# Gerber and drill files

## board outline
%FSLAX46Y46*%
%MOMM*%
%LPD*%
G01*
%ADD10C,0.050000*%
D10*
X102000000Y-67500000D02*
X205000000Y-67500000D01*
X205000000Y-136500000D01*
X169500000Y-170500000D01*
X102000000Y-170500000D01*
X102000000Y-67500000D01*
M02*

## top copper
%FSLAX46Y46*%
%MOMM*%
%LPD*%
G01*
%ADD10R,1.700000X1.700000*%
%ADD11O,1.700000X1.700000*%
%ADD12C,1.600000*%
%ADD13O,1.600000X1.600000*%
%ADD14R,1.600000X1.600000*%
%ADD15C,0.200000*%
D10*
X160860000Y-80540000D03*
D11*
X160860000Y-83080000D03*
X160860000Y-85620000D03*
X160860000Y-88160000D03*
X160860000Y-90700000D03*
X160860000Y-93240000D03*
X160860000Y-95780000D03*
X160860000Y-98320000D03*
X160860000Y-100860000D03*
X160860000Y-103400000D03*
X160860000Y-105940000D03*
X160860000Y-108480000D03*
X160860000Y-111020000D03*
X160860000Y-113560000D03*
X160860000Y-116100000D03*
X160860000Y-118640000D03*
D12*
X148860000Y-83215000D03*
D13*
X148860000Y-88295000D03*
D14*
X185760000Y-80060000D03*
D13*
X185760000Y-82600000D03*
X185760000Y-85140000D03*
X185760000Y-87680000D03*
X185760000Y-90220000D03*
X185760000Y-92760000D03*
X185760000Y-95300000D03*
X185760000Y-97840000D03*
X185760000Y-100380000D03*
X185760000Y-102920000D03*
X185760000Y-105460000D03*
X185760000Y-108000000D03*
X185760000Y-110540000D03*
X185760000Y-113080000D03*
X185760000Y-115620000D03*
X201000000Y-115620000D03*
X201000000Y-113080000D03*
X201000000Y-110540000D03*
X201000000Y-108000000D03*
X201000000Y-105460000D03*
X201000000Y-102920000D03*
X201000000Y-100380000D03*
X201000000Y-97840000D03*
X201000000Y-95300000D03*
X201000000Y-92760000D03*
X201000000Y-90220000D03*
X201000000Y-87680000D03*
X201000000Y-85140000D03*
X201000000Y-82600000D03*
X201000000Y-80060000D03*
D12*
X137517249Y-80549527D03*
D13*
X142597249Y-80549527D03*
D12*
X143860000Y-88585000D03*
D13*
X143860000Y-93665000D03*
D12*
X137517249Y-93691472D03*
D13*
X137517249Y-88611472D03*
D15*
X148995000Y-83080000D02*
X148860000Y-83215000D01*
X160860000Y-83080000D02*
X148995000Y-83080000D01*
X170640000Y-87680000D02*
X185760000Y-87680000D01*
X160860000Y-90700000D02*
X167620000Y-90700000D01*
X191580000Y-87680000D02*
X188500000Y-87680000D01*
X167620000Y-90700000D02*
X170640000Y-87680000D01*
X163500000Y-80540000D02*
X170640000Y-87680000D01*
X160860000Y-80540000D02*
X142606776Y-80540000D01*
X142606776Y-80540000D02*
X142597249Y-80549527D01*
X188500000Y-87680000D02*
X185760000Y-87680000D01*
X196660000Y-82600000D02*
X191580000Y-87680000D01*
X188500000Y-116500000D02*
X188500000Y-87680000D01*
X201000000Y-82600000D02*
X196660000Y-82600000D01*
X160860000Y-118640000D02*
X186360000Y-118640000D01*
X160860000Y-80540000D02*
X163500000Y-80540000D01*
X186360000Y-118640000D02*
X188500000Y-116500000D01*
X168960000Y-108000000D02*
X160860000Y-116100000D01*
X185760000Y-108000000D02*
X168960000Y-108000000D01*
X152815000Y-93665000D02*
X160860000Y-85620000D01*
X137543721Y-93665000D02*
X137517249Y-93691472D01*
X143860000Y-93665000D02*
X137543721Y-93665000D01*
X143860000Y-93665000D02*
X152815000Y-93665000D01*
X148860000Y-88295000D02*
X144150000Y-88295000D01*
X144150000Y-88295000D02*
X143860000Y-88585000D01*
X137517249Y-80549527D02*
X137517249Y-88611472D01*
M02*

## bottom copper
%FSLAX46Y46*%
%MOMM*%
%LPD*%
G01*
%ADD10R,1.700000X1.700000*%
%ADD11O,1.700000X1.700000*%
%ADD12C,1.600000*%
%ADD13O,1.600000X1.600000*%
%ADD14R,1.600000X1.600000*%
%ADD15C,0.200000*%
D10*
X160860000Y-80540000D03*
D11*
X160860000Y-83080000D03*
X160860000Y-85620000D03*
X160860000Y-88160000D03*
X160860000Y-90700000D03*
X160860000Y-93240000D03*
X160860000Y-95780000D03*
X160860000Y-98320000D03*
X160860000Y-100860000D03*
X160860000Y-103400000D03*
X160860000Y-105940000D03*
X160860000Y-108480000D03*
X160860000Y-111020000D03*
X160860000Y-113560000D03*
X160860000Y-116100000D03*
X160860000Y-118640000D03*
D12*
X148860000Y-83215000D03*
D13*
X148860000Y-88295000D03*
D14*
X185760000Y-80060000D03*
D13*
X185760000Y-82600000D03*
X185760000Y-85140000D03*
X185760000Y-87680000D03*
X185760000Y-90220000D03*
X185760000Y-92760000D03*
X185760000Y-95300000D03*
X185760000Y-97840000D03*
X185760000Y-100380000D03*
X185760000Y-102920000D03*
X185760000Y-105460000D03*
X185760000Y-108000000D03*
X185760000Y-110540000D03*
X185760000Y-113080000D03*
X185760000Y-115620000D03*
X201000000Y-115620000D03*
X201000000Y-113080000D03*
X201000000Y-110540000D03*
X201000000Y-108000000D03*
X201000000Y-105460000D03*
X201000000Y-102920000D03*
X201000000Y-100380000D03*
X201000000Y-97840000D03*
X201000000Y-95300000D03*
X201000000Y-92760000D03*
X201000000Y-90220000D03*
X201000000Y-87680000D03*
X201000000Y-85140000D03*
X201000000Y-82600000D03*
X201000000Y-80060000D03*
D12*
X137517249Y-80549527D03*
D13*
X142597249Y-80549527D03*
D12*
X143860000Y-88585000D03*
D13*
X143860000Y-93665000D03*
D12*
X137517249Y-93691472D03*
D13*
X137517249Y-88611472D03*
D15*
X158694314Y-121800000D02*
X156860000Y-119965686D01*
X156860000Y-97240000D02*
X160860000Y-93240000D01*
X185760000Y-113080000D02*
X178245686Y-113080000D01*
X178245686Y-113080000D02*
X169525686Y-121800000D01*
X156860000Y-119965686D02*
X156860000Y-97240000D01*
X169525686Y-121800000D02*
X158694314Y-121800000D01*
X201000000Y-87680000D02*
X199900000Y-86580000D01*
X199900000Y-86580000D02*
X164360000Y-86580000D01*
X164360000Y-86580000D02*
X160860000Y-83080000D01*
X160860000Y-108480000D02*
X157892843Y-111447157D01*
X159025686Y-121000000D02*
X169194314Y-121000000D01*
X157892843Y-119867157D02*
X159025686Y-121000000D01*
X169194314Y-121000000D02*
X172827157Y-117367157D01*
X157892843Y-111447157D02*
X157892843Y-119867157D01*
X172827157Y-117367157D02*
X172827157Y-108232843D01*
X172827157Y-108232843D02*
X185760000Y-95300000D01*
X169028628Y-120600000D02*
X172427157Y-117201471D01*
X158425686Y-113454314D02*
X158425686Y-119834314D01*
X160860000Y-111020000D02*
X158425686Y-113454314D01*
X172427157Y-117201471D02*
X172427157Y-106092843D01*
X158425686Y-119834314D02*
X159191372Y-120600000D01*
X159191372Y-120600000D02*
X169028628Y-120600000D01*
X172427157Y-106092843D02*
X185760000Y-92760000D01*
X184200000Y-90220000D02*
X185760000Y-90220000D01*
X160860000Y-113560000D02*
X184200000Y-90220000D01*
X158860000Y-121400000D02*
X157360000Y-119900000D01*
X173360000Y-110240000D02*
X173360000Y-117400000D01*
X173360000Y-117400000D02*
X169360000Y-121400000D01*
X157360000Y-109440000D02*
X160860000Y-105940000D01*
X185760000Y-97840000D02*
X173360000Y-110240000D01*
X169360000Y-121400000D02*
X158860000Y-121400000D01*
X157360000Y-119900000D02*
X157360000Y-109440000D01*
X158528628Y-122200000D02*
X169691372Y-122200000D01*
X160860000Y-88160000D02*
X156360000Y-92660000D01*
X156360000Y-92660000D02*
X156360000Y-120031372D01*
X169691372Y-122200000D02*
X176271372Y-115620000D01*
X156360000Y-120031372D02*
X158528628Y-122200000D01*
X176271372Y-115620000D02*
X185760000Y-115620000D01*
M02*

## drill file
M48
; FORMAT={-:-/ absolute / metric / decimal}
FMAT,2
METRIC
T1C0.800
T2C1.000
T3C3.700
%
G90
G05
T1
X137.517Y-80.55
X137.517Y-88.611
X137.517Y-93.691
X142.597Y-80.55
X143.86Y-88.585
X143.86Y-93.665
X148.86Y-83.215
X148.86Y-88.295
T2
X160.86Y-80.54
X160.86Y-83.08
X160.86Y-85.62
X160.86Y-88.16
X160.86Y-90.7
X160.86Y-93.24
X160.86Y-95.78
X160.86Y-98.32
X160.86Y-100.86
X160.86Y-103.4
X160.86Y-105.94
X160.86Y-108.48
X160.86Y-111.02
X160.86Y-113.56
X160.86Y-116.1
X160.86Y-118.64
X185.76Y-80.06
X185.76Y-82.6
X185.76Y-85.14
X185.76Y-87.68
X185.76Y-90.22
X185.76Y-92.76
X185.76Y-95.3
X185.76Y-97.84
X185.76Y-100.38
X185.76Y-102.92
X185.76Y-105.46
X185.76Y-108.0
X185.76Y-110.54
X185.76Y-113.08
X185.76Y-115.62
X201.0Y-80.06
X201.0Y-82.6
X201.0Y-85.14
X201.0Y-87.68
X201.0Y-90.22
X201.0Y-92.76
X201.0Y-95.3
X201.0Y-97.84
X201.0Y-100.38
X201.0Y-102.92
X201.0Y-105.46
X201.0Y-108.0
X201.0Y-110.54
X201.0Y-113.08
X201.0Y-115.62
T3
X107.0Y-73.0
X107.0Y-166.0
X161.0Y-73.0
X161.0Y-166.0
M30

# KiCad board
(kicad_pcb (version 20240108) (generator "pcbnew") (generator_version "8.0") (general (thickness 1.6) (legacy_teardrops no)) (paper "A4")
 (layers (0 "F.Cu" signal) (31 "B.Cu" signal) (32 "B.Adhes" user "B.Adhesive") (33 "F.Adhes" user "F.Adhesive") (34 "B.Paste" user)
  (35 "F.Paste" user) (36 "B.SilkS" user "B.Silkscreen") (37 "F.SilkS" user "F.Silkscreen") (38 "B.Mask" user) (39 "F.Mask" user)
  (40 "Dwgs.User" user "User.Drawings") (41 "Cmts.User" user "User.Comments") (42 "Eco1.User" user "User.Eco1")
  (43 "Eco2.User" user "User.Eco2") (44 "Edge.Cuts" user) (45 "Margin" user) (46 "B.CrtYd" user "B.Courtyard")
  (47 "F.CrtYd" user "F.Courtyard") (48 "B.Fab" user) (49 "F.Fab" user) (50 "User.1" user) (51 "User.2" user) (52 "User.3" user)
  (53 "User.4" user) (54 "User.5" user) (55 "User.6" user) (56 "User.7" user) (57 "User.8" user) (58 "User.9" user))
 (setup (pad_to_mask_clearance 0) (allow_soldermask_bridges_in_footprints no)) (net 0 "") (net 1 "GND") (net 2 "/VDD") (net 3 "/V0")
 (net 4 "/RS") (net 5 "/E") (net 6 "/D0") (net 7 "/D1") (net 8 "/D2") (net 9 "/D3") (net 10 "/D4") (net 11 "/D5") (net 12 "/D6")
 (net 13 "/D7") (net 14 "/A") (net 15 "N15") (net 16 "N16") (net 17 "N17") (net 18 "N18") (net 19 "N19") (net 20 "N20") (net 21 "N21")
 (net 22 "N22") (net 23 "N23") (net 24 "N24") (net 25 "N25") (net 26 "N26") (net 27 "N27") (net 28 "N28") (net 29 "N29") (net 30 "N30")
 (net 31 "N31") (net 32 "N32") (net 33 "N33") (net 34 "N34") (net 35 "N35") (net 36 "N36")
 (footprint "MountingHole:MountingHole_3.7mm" (layer "F.Cu") (at 107 166)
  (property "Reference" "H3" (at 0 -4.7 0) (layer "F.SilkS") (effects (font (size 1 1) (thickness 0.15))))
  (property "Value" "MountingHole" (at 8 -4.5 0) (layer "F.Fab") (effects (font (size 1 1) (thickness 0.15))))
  (pad "" np_thru_hole circle (at 0 0) (size 3.7 3.7) (drill 3.7) (layers "*.Cu" "*.Mask")))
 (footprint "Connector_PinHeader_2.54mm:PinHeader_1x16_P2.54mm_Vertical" (layer "F.Cu") (at 160.86 80.54)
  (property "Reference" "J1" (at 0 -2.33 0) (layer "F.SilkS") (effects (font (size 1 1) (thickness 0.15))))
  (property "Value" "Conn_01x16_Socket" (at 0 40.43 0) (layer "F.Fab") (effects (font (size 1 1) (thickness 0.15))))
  (pad "1" thru_hole rect (at 0 0) (size 1.7 1.7) (drill 1) (layers "*.Cu" "*.Mask") (remove_unused_layers no) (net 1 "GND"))
  (pad "2" thru_hole oval (at 0 2.54) (size 1.7 1.7) (drill 1) (layers "*.Cu" "*.Mask") (remove_unused_layers no) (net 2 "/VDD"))
  (pad "3" thru_hole oval (at 0 5.08) (size 1.7 1.7) (drill 1) (layers "*.Cu" "*.Mask") (remove_unused_layers no) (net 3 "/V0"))
  (pad "4" thru_hole oval (at 0 7.62) (size 1.7 1.7) (drill 1) (layers "*.Cu" "*.Mask") (remove_unused_layers no) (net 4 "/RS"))
  (pad "5" thru_hole oval (at 0 10.16) (size 1.7 1.7) (drill 1) (layers "*.Cu" "*.Mask") (remove_unused_layers no) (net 1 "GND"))
  (pad "6" thru_hole oval (at 0 12.7) (size 1.7 1.7) (drill 1) (layers "*.Cu" "*.Mask") (remove_unused_layers no) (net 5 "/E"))
  (pad "7" thru_hole oval (at 0 15.24) (size 1.7 1.7) (drill 1) (layers "*.Cu" "*.Mask") (remove_unused_layers no) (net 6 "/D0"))
  (pad "8" thru_hole oval (at 0 17.78) (size 1.7 1.7) (drill 1) (layers "*.Cu" "*.Mask") (remove_unused_layers no) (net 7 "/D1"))
  (pad "9" thru_hole oval (at 0 20.32) (size 1.7 1.7) (drill 1) (layers "*.Cu" "*.Mask") (remove_unused_layers no) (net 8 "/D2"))
  (pad "10" thru_hole oval (at 0 22.86) (size 1.7 1.7) (drill 1) (layers "*.Cu" "*.Mask") (remove_unused_layers no) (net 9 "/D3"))
  (pad "11" thru_hole oval (at 0 25.4) (size 1.7 1.7) (drill 1) (layers "*.Cu" "*.Mask") (remove_unused_layers no) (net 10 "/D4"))
  (pad "12" thru_hole oval (at 0 27.94) (size 1.7 1.7) (drill 1) (layers "*.Cu" "*.Mask") (remove_unused_layers no) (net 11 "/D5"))
  (pad "13" thru_hole oval (at 0 30.48) (size 1.7 1.7) (drill 1) (layers "*.Cu" "*.Mask") (remove_unused_layers no) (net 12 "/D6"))
  (pad "14" thru_hole oval (at 0 33.02) (size 1.7 1.7) (drill 1) (layers "*.Cu" "*.Mask") (remove_unused_layers no) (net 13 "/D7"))
  (pad "15" thru_hole oval (at 0 35.56) (size 1.7 1.7) (drill 1) (layers "*.Cu" "*.Mask") (remove_unused_layers no) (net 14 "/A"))
  (pad "16" thru_hole oval (at 0 38.1) (size 1.7 1.7) (drill 1) (layers "*.Cu" "*.Mask") (remove_unused_layers no) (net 1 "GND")))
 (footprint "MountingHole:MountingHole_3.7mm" (layer "F.Cu") (at 161 166)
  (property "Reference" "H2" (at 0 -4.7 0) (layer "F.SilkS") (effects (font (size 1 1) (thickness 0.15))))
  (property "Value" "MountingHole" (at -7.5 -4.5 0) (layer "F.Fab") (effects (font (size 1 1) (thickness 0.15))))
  (pad "" np_thru_hole circle (at 0 0) (size 3.7 3.7) (drill 3.7) (layers "*.Cu" "*.Mask")))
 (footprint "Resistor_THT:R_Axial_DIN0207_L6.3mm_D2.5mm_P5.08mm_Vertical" (layer "F.Cu") (at 148.86 83.215 -90)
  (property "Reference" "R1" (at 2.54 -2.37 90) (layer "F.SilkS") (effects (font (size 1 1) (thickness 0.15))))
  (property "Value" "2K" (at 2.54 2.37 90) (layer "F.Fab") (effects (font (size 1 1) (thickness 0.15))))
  (pad "1" thru_hole circle (at 0 0 270) (size 1.6 1.6) (drill 0.8) (layers "*.Cu" "*.Mask") (remove_unused_layers no) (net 2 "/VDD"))
  (pad "2" thru_hole oval (at 5.08 0 270) (size 1.6 1.6) (drill 0.8) (layers "*.Cu" "*.Mask") (remove_unused_layers no) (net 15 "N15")))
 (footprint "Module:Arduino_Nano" (layer "F.Cu") (at 185.76 80.06)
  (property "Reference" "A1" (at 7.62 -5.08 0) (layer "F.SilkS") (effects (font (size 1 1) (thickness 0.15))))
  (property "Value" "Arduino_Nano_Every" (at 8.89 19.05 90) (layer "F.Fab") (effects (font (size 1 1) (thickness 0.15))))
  (pad "1" thru_hole rect (at 0 0) (size 1.6 1.6) (drill 1) (layers "*.Cu" "*.Mask") (remove_unused_layers no) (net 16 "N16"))
  (pad "2" thru_hole oval (at 0 2.54) (size 1.6 1.6) (drill 1) (layers "*.Cu" "*.Mask") (remove_unused_layers no) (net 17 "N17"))
  (pad "3" thru_hole oval (at 0 5.08) (size 1.6 1.6) (drill 1) (layers "*.Cu" "*.Mask") (remove_unused_layers no) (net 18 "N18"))
  (pad "4" thru_hole oval (at 0 7.62) (size 1.6 1.6) (drill 1) (layers "*.Cu" "*.Mask") (remove_unused_layers no) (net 1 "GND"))
  (pad "5" thru_hole oval (at 0 10.16) (size 1.6 1.6) (drill 1) (layers "*.Cu" "*.Mask") (remove_unused_layers no) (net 13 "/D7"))
  (pad "6" thru_hole oval (at 0 12.7) (size 1.6 1.6) (drill 1) (layers "*.Cu" "*.Mask") (remove_unused_layers no) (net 12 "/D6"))
  (pad "7" thru_hole oval (at 0 15.24) (size 1.6 1.6) (drill 1) (layers "*.Cu" "*.Mask") (remove_unused_layers no) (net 11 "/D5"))
  (pad "8" thru_hole oval (at 0 17.78) (size 1.6 1.6) (drill 1) (layers "*.Cu" "*.Mask") (remove_unused_layers no) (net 10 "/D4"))
  (pad "9" thru_hole oval (at 0 20.32) (size 1.6 1.6) (drill 1) (layers "*.Cu" "*.Mask") (remove_unused_layers no) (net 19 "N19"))
  (pad "10" thru_hole oval (at 0 22.86) (size 1.6 1.6) (drill 1) (layers "*.Cu" "*.Mask") (remove_unused_layers no) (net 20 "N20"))
  (pad "11" thru_hole oval (at 0 25.4) (size 1.6 1.6) (drill 1) (layers "*.Cu" "*.Mask") (remove_unused_layers no) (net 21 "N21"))
  (pad "12" thru_hole oval (at 0 27.94) (size 1.6 1.6) (drill 1) (layers "*.Cu" "*.Mask") (remove_unused_layers no) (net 14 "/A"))
  (pad "13" thru_hole oval (at 0 30.48) (size 1.6 1.6) (drill 1) (layers "*.Cu" "*.Mask") (remove_unused_layers no) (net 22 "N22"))
  (pad "14" thru_hole oval (at 0 33.02) (size 1.6 1.6) (drill 1) (layers "*.Cu" "*.Mask") (remove_unused_layers no) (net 5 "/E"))
  (pad "15" thru_hole oval (at 0 35.56) (size 1.6 1.6) (drill 1) (layers "*.Cu" "*.Mask") (remove_unused_layers no) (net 4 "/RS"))
  (pad "16" thru_hole oval (at 15.24 35.56) (size 1.6 1.6) (drill 1) (layers "*.Cu" "*.Mask") (remove_unused_layers no) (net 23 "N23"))
  (pad "17" thru_hole oval (at 15.24 33.02) (size 1.6 1.6) (drill 1) (layers "*.Cu" "*.Mask") (remove_unused_layers no) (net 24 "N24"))
  (pad "18" thru_hole oval (at 15.24 30.48) (size 1.6 1.6) (drill 1) (layers "*.Cu" "*.Mask") (remove_unused_layers no) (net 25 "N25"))
  (pad "19" thru_hole oval (at 15.24 27.94) (size 1.6 1.6) (drill 1) (layers "*.Cu" "*.Mask") (remove_unused_layers no) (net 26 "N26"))
  (pad "20" thru_hole oval (at 15.24 25.4) (size 1.6 1.6) (drill 1) (layers "*.Cu" "*.Mask") (remove_unused_layers no) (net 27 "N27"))
  (pad "21" thru_hole oval (at 15.24 22.86) (size 1.6 1.6) (drill 1) (layers "*.Cu" "*.Mask") (remove_unused_layers no) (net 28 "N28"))
  (pad "22" thru_hole oval (at 15.24 20.32) (size 1.6 1.6) (drill 1) (layers "*.Cu" "*.Mask") (remove_unused_layers no) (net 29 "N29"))
  (pad "23" thru_hole oval (at 15.24 17.78) (size 1.6 1.6) (drill 1) (layers "*.Cu" "*.Mask") (remove_unused_layers no) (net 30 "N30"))
  (pad "24" thru_hole oval (at 15.24 15.24) (size 1.6 1.6) (drill 1) (layers "*.Cu" "*.Mask") (remove_unused_layers no) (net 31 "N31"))
  (pad "25" thru_hole oval (at 15.24 12.7) (size 1.6 1.6) (drill 1) (layers "*.Cu" "*.Mask") (remove_unused_layers no) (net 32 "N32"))
  (pad "26" thru_hole oval (at 15.24 10.16) (size 1.6 1.6) (drill 1) (layers "*.Cu" "*.Mask") (remove_unused_layers no) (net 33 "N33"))
  (pad "27" thru_hole oval (at 15.24 7.62) (size 1.6 1.6) (drill 1) (layers "*.Cu" "*.Mask") (remove_unused_layers no) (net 2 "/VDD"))
  (pad "28" thru_hole oval (at 15.24 5.08) (size 1.6 1.6) (drill 1) (layers "*.Cu" "*.Mask") (remove_unused_layers no) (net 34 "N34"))
  (pad "29" thru_hole oval (at 15.24 2.54) (size 1.6 1.6) (drill 1) (layers "*.Cu" "*.Mask") (remove_unused_layers no) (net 1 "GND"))
  (pad "30" thru_hole oval (at 15.24 0) (size 1.6 1.6) (drill 1) (layers "*.Cu" "*.Mask") (remove_unused_layers no) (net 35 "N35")))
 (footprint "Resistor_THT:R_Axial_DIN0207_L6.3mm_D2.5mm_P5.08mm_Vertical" (layer "F.Cu") (at 137.517249 80.549527)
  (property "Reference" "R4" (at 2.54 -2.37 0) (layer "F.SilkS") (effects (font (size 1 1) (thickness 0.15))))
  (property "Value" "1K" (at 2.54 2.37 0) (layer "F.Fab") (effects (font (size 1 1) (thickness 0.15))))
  (pad "1" thru_hole circle (at 0 0) (size 1.6 1.6) (drill 0.8) (layers "*.Cu" "*.Mask") (remove_unused_layers no) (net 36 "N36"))
  (pad "2" thru_hole oval (at 5.08 0) (size 1.6 1.6) (drill 0.8) (layers "*.Cu" "*.Mask") (remove_unused_layers no) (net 1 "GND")))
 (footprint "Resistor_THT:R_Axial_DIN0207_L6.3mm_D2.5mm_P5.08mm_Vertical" (layer "F.Cu") (at 143.86 88.585 -90)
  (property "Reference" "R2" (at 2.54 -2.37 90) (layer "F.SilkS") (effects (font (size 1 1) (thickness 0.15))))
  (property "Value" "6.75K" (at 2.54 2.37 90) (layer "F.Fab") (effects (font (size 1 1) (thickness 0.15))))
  (pad "1" thru_hole circle (at 0 0 270) (size 1.6 1.6) (drill 0.8) (layers "*.Cu" "*.Mask") (remove_unused_layers no) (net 15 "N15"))
  (pad "2" thru_hole oval (at 5.08 0 270) (size 1.6 1.6) (drill 0.8) (layers "*.Cu" "*.Mask") (remove_unused_layers no) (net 3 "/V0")))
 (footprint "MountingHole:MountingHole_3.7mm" (layer "F.Cu") (at 107 73)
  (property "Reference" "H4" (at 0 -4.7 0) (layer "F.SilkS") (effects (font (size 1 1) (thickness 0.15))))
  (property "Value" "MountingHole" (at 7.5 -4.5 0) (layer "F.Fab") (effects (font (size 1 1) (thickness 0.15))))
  (pad "" np_thru_hole circle (at 0 0) (size 3.7 3.7) (drill 3.7) (layers "*.Cu" "*.Mask")))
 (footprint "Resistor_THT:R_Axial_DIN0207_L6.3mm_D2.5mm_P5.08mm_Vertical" (layer "F.Cu") (at 137.517249 93.691472 90)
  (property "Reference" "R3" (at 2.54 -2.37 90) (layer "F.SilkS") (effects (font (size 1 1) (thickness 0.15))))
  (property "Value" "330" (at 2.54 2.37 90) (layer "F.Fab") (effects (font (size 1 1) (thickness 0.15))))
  (pad "1" thru_hole circle (at 0 0 90) (size 1.6 1.6) (drill 0.8) (layers "*.Cu" "*.Mask") (remove_unused_layers no) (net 3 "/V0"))
  (pad "2" thru_hole oval (at 5.08 0 90) (size 1.6 1.6) (drill 0.8) (layers "*.Cu" "*.Mask") (remove_unused_layers no) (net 36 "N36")))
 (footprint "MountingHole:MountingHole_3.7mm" (layer "F.Cu") (at 161 73)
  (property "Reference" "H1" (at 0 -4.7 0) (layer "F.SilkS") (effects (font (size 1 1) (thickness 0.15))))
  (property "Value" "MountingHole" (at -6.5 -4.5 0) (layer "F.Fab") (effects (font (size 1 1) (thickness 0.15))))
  (pad "" np_thru_hole circle (at 0 0) (size 3.7 3.7) (drill 3.7) (layers "*.Cu" "*.Mask")))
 (gr_poly
  (pts (xy 102 67.5) (xy 205 67.5) (xy 205 136.5) (xy 169.5 170.5) (xy 102 170.5)) (stroke (width 0.05) (type solid)) (fill none)
  (layer "Edge.Cuts"))
 (segment (start 158.694314 121.8) (end 156.86 119.965686) (width 0.2) (layer "B.Cu") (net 5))
 (segment (start 156.86 97.24) (end 160.86 93.24) (width 0.2) (layer "B.Cu") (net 5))
 (segment (start 185.76 113.08) (end 178.245686 113.08) (width 0.2) (layer "B.Cu") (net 5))
 (segment (start 178.245686 113.08) (end 169.525686 121.8) (width 0.2) (layer "B.Cu") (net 5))
 (segment (start 156.86 119.965686) (end 156.86 97.24) (width 0.2) (layer "B.Cu") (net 5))
 (segment (start 169.525686 121.8) (end 158.694314 121.8) (width 0.2) (layer "B.Cu") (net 5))
 (segment (start 148.995 83.08) (end 148.86 83.215) (width 0.2) (layer "F.Cu") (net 2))
 (segment (start 160.86 83.08) (end 148.995 83.08) (width 0.2) (layer "F.Cu") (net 2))
 (segment (start 201 87.68) (end 199.9 86.58) (width 0.2) (layer "B.Cu") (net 2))
 (segment (start 199.9 86.58) (end 164.36 86.58) (width 0.2) (layer "B.Cu") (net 2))
 (segment (start 164.36 86.58) (end 160.86 83.08) (width 0.2) (layer "B.Cu") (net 2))
 (segment (start 170.64 87.68) (end 185.76 87.68) (width 0.2) (layer "F.Cu") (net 1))
 (segment (start 160.86 90.7) (end 167.62 90.7) (width 0.2) (layer "F.Cu") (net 1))
 (segment (start 191.58 87.68) (end 188.5 87.68) (width 0.2) (layer "F.Cu") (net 1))
 (segment (start 167.62 90.7) (end 170.64 87.68) (width 0.2) (layer "F.Cu") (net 1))
 (segment (start 163.5 80.54) (end 170.64 87.68) (width 0.2) (layer "F.Cu") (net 1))
 (segment (start 160.86 80.54) (end 142.606776 80.54) (width 0.2) (layer "F.Cu") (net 1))
 (segment (start 142.606776 80.54) (end 142.597249 80.549527) (width 0.2) (layer "F.Cu") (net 1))
 (segment (start 188.5 87.68) (end 185.76 87.68) (width 0.2) (layer "F.Cu") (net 1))
 (segment (start 196.66 82.6) (end 191.58 87.68) (width 0.2) (layer "F.Cu") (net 1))
 (segment (start 188.5 116.5) (end 188.5 87.68) (width 0.2) (layer "F.Cu") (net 1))
 (segment (start 201 82.6) (end 196.66 82.6) (width 0.2) (layer "F.Cu") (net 1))
 (segment (start 160.86 118.64) (end 186.36 118.64) (width 0.2) (layer "F.Cu") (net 1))
 (segment (start 160.86 80.54) (end 163.5 80.54) (width 0.2) (layer "F.Cu") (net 1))
 (segment (start 186.36 118.64) (end 188.5 116.5) (width 0.2) (layer "F.Cu") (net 1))
 (segment (start 160.86 108.48) (end 157.892843 111.447157) (width 0.2) (layer "B.Cu") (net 11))
 (segment (start 159.025686 121) (end 169.194314 121) (width 0.2) (layer "B.Cu") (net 11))
 (segment (start 157.892843 119.867157) (end 159.025686 121) (width 0.2) (layer "B.Cu") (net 11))
 (segment (start 169.194314 121) (end 172.827157 117.367157) (width 0.2) (layer "B.Cu") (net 11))
 (segment (start 157.892843 111.447157) (end 157.892843 119.867157) (width 0.2) (layer "B.Cu") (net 11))
 (segment (start 172.827157 117.367157) (end 172.827157 108.232843) (width 0.2) (layer "B.Cu") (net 11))
 (segment (start 172.827157 108.232843) (end 185.76 95.3) (width 0.2) (layer "B.Cu") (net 11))
 (segment (start 169.028628 120.6) (end 172.427157 117.201471) (width 0.2) (layer "B.Cu") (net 12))
 (segment (start 158.425686 113.454314) (end 158.425686 119.834314) (width 0.2) (layer "B.Cu") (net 12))
 (segment (start 160.86 111.02) (end 158.425686 113.454314) (width 0.2) (layer "B.Cu") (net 12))
 (segment (start 172.427157 117.201471) (end 172.427157 106.092843) (width 0.2) (layer "B.Cu") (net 12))
 (segment (start 158.425686 119.834314) (end 159.191372 120.6) (width 0.2) (layer "B.Cu") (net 12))
 (segment (start 159.191372 120.6) (end 169.028628 120.6) (width 0.2) (layer "B.Cu") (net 12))
 (segment (start 172.427157 106.092843) (end 185.76 92.76) (width 0.2) (layer "B.Cu") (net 12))
 (segment (start 184.2 90.22) (end 185.76 90.22) (width 0.2) (layer "B.Cu") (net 13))
 (segment (start 160.86 113.56) (end 184.2 90.22) (width 0.2) (layer "B.Cu") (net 13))
 (segment (start 158.86 121.4) (end 157.36 119.9) (width 0.2) (layer "B.Cu") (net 10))
 (segment (start 173.36 110.24) (end 173.36 117.4) (width 0.2) (layer "B.Cu") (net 10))
 (segment (start 173.36 117.4) (end 169.36 121.4) (width 0.2) (layer "B.Cu") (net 10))
 (segment (start 157.36 109.44) (end 160.86 105.94) (width 0.2) (layer "B.Cu") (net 10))
 (segment (start 185.76 97.84) (end 173.36 110.24) (width 0.2) (layer "B.Cu") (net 10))
 (segment (start 169.36 121.4) (end 158.86 121.4) (width 0.2) (layer "B.Cu") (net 10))
 (segment (start 157.36 119.9) (end 157.36 109.44) (width 0.2) (layer "B.Cu") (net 10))
 (segment (start 168.96 108) (end 160.86 116.1) (width 0.2) (layer "F.Cu") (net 14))
 (segment (start 185.76 108) (end 168.96 108) (width 0.2) (layer "F.Cu") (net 14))
 (segment (start 158.528628 122.2) (end 169.691372 122.2) (width 0.2) (layer "B.Cu") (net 4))
 (segment (start 160.86 88.16) (end 156.36 92.66) (width 0.2) (layer "B.Cu") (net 4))
 (segment (start 156.36 92.66) (end 156.36 120.031372) (width 0.2) (layer "B.Cu") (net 4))
 (segment (start 169.691372 122.2) (end 176.271372 115.62) (width 0.2) (layer "B.Cu") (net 4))
 (segment (start 156.36 120.031372) (end 158.528628 122.2) (width 0.2) (layer "B.Cu") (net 4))
 (segment (start 176.271372 115.62) (end 185.76 115.62) (width 0.2) (layer "B.Cu") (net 4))
 (segment (start 152.815 93.665) (end 160.86 85.62) (width 0.2) (layer "F.Cu") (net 3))
 (segment (start 137.543721 93.665) (end 137.517249 93.691472) (width 0.2) (layer "F.Cu") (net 3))
 (segment (start 143.86 93.665) (end 137.543721 93.665) (width 0.2) (layer "F.Cu") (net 3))
 (segment (start 143.86 93.665) (end 152.815 93.665) (width 0.2) (layer "F.Cu") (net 3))
 (segment (start 148.86 88.295) (end 144.15 88.295) (width 0.2) (layer "F.Cu") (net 15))
 (segment (start 144.15 88.295) (end 143.86 88.585) (width 0.2) (layer "F.Cu") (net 15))
 (segment (start 137.517249 80.549527) (end 137.517249 88.611472) (width 0.2) (layer "F.Cu") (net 36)))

